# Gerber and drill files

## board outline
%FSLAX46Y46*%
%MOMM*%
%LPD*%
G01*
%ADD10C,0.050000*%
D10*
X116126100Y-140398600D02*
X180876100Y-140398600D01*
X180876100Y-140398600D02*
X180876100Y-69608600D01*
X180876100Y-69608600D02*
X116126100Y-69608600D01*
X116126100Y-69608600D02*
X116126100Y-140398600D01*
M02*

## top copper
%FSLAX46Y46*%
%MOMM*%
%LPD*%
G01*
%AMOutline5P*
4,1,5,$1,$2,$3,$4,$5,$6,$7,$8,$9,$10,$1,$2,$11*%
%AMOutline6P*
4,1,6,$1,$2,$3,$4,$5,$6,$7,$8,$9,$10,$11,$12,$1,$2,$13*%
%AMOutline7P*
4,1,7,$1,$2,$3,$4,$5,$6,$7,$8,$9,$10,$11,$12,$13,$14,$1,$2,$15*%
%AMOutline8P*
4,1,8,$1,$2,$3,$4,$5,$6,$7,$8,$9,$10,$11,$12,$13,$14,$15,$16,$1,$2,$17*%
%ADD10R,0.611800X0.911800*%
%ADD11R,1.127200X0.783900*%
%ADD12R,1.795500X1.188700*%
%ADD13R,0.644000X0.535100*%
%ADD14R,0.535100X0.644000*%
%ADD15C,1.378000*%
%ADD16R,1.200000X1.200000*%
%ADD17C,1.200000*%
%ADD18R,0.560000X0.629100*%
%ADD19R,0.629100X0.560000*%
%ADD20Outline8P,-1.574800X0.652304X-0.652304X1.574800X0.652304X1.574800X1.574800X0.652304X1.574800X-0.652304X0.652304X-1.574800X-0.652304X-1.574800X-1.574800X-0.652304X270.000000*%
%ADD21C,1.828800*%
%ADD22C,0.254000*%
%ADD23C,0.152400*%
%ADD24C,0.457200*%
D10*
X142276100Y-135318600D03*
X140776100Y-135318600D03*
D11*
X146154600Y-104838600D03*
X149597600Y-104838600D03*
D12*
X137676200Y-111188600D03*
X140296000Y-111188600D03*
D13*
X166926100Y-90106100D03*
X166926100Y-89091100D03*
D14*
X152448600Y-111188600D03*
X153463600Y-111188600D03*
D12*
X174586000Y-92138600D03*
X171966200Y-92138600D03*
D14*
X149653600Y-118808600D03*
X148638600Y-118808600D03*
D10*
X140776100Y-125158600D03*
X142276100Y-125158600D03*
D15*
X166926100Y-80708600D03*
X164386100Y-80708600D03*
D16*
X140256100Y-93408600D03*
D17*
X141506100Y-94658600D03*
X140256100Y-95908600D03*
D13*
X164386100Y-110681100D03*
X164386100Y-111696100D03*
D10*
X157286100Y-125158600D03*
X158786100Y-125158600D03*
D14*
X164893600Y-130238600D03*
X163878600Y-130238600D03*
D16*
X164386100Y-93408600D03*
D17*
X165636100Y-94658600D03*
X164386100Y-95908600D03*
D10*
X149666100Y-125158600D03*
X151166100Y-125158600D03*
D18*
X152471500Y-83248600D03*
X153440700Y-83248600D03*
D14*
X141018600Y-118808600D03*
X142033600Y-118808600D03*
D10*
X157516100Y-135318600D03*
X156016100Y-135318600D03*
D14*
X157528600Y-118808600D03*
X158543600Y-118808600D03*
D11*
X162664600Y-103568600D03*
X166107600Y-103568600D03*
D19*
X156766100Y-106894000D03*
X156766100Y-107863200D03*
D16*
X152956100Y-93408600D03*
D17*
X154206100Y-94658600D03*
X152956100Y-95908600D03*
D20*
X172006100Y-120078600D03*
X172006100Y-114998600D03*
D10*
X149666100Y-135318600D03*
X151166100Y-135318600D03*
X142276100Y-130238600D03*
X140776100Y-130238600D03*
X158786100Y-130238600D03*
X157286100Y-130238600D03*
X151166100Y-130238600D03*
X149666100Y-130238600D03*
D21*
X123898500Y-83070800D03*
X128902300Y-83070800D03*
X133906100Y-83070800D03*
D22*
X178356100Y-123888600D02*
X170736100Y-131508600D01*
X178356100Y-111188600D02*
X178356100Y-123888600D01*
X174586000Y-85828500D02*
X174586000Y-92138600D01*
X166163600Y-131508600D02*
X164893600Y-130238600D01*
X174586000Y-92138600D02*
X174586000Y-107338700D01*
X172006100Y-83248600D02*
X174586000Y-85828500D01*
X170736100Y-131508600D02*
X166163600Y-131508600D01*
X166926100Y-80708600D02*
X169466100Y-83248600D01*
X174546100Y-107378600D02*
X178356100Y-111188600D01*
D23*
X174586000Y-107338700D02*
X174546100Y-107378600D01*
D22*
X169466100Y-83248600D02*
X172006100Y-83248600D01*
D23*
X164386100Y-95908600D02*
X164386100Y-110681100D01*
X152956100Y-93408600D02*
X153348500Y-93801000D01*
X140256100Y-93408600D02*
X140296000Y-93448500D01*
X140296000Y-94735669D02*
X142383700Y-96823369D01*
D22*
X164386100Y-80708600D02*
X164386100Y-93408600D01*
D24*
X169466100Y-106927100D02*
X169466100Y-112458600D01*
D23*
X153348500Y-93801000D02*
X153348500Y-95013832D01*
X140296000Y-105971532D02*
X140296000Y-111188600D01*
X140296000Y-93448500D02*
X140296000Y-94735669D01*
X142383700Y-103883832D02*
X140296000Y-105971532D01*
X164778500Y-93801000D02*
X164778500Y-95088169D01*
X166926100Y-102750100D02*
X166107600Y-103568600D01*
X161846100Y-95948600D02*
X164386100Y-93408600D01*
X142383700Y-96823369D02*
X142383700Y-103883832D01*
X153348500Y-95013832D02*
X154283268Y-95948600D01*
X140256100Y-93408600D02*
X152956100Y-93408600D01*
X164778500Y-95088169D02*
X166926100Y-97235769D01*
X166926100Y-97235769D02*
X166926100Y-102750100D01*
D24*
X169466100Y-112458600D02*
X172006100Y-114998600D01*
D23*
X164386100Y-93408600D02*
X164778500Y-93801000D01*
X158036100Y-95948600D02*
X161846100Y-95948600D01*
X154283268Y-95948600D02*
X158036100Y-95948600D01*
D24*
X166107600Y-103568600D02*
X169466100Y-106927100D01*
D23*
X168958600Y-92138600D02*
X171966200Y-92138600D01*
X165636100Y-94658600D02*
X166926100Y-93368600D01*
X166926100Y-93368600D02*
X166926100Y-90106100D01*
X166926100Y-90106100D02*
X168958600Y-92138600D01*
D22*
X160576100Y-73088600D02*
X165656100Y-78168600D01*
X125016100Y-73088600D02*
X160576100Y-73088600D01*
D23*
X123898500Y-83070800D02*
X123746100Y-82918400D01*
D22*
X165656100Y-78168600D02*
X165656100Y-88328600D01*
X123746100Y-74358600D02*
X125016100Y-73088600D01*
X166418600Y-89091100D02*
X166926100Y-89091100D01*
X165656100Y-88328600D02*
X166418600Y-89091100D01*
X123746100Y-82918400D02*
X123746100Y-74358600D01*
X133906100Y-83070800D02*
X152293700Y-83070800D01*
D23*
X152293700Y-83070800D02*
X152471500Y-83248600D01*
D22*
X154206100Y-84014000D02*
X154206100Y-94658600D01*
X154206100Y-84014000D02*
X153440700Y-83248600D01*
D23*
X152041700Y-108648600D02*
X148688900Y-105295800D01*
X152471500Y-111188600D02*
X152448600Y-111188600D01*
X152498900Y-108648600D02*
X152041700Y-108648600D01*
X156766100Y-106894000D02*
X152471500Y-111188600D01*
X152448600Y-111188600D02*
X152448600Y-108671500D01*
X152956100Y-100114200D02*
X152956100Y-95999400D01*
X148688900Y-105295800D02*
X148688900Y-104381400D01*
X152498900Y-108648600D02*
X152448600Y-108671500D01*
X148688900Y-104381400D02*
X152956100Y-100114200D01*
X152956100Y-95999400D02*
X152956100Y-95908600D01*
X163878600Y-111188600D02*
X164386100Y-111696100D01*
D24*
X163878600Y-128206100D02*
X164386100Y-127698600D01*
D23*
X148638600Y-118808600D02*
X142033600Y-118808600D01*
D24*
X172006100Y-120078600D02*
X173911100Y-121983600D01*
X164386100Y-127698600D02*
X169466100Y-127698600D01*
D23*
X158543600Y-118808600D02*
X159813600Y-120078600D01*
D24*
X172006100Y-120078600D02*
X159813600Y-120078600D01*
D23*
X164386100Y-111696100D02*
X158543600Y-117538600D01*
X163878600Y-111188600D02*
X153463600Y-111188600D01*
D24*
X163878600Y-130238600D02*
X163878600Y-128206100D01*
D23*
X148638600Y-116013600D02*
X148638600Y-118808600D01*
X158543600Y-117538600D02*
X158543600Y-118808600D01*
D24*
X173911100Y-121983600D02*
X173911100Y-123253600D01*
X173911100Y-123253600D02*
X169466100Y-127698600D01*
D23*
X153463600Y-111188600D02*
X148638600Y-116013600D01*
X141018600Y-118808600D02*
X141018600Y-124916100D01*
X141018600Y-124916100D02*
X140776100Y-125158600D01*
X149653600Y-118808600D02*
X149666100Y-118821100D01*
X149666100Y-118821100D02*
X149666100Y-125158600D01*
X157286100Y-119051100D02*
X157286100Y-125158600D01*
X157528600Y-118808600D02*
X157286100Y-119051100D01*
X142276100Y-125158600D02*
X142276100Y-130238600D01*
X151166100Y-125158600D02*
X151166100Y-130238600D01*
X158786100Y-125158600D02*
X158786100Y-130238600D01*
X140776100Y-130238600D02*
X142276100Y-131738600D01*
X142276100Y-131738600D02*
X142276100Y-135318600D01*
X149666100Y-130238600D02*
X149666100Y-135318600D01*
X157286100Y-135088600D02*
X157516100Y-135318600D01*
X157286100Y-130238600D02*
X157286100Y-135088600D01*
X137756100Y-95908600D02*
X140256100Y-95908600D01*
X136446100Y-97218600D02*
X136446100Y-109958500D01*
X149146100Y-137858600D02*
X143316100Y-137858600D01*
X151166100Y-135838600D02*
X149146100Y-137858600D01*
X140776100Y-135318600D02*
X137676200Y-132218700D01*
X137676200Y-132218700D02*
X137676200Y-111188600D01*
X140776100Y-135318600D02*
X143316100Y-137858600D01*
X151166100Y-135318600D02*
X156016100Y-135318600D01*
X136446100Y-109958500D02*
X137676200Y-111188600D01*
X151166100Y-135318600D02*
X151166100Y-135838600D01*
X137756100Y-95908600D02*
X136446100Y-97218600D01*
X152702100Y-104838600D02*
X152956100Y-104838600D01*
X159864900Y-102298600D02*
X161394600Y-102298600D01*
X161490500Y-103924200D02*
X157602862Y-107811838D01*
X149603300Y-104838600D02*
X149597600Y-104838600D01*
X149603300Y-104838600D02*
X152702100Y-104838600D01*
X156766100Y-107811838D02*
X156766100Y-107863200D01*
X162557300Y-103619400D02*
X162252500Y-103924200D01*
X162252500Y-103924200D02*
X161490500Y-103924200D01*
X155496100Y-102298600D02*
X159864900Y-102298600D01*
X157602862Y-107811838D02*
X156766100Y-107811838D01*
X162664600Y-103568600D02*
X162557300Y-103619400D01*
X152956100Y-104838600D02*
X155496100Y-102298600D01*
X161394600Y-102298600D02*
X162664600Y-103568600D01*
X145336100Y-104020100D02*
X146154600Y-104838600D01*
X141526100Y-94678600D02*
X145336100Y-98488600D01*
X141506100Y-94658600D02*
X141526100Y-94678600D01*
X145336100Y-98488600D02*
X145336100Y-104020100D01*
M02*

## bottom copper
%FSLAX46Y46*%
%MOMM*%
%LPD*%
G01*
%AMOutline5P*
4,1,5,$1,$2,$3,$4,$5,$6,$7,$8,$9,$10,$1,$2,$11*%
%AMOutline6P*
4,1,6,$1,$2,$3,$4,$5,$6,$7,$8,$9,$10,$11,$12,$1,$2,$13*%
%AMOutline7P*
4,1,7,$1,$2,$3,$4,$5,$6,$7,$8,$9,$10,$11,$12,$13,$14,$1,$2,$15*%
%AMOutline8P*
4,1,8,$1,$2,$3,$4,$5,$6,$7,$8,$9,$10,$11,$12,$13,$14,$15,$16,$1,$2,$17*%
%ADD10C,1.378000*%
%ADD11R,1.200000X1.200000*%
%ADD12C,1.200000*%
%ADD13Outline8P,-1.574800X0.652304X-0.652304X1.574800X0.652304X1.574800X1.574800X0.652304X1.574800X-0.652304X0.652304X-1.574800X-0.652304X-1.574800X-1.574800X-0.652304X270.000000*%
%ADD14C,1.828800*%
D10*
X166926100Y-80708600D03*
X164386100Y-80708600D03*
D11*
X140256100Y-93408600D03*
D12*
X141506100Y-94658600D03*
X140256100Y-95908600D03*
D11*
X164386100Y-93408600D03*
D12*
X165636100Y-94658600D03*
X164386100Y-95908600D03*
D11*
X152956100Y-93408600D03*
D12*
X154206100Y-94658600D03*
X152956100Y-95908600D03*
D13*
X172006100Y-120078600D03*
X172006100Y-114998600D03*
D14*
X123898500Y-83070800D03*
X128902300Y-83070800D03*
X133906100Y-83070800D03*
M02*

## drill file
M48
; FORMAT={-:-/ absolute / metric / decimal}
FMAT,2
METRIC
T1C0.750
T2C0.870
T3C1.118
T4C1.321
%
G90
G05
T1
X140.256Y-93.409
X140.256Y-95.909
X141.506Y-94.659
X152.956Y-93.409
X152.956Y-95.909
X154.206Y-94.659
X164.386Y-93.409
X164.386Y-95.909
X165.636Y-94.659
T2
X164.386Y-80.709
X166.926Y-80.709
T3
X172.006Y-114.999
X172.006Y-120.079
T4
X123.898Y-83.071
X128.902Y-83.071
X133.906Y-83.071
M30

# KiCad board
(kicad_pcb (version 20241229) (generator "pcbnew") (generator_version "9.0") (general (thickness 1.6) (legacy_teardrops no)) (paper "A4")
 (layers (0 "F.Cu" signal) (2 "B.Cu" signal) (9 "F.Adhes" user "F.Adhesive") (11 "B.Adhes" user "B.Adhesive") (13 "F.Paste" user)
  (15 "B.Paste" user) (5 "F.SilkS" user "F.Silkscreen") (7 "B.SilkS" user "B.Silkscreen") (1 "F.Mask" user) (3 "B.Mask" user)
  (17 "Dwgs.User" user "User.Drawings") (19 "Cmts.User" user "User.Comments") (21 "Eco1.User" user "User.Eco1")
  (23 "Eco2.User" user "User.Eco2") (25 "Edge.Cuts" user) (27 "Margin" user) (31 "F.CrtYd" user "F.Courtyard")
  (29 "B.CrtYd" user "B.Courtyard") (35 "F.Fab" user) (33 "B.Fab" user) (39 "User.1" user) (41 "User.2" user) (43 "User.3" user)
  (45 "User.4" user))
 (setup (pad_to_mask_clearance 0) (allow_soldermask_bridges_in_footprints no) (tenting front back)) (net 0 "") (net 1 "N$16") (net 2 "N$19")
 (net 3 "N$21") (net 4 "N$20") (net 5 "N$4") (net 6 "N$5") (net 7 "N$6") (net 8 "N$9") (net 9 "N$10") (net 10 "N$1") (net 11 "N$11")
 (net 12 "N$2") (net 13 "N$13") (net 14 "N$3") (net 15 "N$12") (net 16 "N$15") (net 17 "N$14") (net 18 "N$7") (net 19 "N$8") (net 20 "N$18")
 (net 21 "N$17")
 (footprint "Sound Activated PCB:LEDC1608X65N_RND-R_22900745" (layer "F.Cu") (at 141.5261 135.3186)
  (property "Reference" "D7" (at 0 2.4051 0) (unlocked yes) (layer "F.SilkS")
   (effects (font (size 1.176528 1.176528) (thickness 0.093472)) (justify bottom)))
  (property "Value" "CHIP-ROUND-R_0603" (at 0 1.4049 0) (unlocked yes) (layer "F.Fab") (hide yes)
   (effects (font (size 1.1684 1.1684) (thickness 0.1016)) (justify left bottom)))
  (pad "A" smd rect (at 0.75 0) (size 0.6118 0.9118) (layers "F.Cu" "F.Mask" "F.Paste") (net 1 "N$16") (solder_mask_margin 0.1016)
   (solder_paste_margin 0) (thermal_bridge_angle 0))
  (pad "C" smd rect (at -0.75 0) (size 0.6118 0.9118) (layers "F.Cu" "F.Mask" "F.Paste") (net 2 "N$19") (solder_mask_margin 0.1016)
   (solder_paste_margin 0) (thermal_bridge_angle 0)))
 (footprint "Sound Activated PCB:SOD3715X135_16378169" (layer "F.Cu") (at 147.8761 104.8386)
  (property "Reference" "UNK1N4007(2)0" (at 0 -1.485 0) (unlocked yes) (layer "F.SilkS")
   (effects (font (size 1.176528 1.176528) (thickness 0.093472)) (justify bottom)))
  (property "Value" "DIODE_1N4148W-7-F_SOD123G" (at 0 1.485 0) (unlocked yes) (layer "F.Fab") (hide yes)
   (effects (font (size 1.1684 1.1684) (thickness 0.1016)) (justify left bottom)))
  (pad "1" smd rect (at -1.7215 0) (size 1.1272 0.7839) (layers "F.Cu" "F.Mask" "F.Paste") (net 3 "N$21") (solder_mask_margin 0.1016)
   (solder_paste_margin 0) (thermal_bridge_angle 0))
  (pad "2" smd rect (at 1.7215 0) (size 1.1272 0.7839) (layers "F.Cu" "F.Mask" "F.Paste") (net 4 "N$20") (solder_mask_margin 0.1016)
   (solder_paste_margin 0) (thermal_bridge_angle 0)))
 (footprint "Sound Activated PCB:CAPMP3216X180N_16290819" (layer "F.Cu") (at 138.9861 111.1886)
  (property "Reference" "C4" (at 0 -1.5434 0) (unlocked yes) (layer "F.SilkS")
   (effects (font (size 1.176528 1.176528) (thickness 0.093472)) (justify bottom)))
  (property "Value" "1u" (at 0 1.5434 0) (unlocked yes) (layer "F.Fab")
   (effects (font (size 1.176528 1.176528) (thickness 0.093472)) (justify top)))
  (pad "1" smd rect (at -1.3099 0) (size 1.7955 1.1887) (layers "F.Cu" "F.Mask" "F.Paste") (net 2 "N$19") (solder_mask_margin 0.1016)
   (solder_paste_margin 0) (thermal_bridge_angle 0))
  (pad "2" smd rect (at 1.3099 0) (size 1.7955 1.1887) (layers "F.Cu" "F.Mask" "F.Paste") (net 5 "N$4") (solder_mask_margin 0.1016)
   (solder_paste_margin 0) (thermal_bridge_angle 0)))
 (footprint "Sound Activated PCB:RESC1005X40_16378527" (layer "F.Cu") (at 166.9261 89.5986 90)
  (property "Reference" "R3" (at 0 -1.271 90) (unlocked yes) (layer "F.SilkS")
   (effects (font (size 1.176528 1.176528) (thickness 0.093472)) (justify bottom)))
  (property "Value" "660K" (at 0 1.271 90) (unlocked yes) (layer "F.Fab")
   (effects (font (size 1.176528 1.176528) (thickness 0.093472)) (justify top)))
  (pad "1" smd rect (at -0.5075 0 90) (size 0.5351 0.644) (layers "F.Cu" "F.Mask" "F.Paste") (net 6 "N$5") (solder_mask_margin 0.1016)
   (solder_paste_margin 0) (thermal_bridge_angle 0))
  (pad "2" smd rect (at 0.5075 0 90) (size 0.5351 0.644) (layers "F.Cu" "F.Mask" "F.Paste") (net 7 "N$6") (solder_mask_margin 0.1016)
   (solder_paste_margin 0) (thermal_bridge_angle 0)))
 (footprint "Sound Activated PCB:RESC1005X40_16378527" (layer "F.Cu") (at 152.9561 111.1886)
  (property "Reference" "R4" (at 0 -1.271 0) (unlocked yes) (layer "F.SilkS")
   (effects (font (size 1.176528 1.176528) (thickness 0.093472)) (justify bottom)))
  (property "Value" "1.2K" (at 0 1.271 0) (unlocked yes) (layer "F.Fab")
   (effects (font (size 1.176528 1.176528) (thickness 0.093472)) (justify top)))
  (pad "1" smd rect (at -0.5075 0) (size 0.5351 0.644) (layers "F.Cu" "F.Mask" "F.Paste") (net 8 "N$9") (solder_mask_margin 0.1016)
   (solder_paste_margin 0) (thermal_bridge_angle 0))
  (pad "2" smd rect (at 0.5075 0) (size 0.5351 0.644) (layers "F.Cu" "F.Mask" "F.Paste") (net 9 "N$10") (solder_mask_margin 0.1016)
   (solder_paste_margin 0) (thermal_bridge_angle 0)))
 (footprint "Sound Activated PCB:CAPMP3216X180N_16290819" (layer "F.Cu") (at 173.2761 92.1386 180)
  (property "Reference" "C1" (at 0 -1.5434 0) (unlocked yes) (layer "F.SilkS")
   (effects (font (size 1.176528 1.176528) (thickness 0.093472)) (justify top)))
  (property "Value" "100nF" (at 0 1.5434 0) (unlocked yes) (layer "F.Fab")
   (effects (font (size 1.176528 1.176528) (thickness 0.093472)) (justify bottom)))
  (pad "1" smd rect (at -1.3099 0 180) (size 1.7955 1.1887) (layers "F.Cu" "F.Mask" "F.Paste") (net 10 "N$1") (solder_mask_margin 0.1016)
   (solder_paste_margin 0) (thermal_bridge_angle 0))
  (pad "2" smd rect (at 1.3099 0 180) (size 1.7955 1.1887) (layers "F.Cu" "F.Mask" "F.Paste") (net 6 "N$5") (solder_mask_margin 0.1016)
   (solder_paste_margin 0) (thermal_bridge_angle 0)))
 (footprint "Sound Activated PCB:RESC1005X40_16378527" (layer "F.Cu") (at 149.1461 118.8086 180)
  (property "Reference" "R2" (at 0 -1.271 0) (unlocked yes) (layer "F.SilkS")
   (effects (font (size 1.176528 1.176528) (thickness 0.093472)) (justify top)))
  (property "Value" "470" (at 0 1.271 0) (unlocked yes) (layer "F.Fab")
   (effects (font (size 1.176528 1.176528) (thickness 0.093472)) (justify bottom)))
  (pad "1" smd rect (at -0.5075 0 180) (size 0.5351 0.644) (layers "F.Cu" "F.Mask" "F.Paste") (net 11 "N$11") (solder_mask_margin 0.1016)
   (solder_paste_margin 0) (thermal_bridge_angle 0))
  (pad "2" smd rect (at 0.5075 0 180) (size 0.5351 0.644) (layers "F.Cu" "F.Mask" "F.Paste") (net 9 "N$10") (solder_mask_margin 0.1016)
   (solder_paste_margin 0) (thermal_bridge_angle 0)))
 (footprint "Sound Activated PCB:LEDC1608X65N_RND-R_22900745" (layer "F.Cu") (at 141.5261 125.1586 180)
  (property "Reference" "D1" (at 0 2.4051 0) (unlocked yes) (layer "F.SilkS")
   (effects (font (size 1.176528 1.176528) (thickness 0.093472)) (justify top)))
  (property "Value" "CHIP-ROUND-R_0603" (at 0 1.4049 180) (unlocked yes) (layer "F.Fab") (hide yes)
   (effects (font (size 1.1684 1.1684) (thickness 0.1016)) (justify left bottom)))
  (pad "A" smd rect (at 0.75 0 180) (size 0.6118 0.9118) (layers "F.Cu" "F.Mask" "F.Paste") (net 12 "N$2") (solder_mask_margin 0.1016)
   (solder_paste_margin 0) (thermal_bridge_angle 0))
  (pad "C" smd rect (at -0.75 0 180) (size 0.6118 0.9118) (layers "F.Cu" "F.Mask" "F.Paste") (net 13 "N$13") (solder_mask_margin 0.1016)
   (solder_paste_margin 0) (thermal_bridge_angle 0)))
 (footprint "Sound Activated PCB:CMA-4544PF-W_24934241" (layer "F.Cu") (at 164.3861 80.7086 90)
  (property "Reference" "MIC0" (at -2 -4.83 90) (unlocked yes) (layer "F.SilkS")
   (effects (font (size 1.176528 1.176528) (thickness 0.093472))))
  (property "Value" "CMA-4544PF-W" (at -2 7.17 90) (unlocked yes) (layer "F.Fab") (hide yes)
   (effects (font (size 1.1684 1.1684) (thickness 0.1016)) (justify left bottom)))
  (pad "1" thru_hole circle (at 0 2.54 90) (size 1.378 1.378) (drill 0.87) (layers "*.Cu" "*.Mask") (remove_unused_layers no) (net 10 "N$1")
   (solder_mask_margin 0.1016) (thermal_bridge_angle 0))
  (pad "2" thru_hole circle (at 0 0 90) (size 1.378 1.378) (drill 0.87) (layers "*.Cu" "*.Mask") (remove_unused_layers no) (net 5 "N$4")
   (solder_mask_margin 0.1016) (thermal_bridge_angle 0)))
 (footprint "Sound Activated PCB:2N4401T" (layer "F.Cu") (at 140.2561 93.4086 -90)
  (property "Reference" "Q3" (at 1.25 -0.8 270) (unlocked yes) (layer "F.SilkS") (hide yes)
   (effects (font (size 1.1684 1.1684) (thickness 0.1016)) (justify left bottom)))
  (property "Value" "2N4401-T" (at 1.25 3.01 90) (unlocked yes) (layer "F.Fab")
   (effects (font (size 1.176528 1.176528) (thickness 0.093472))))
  (pad "1" thru_hole rect (at 0 0 270) (size 1.2 1.2) (drill 0.75) (layers "*.Cu" "*.Mask") (remove_unused_layers no) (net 5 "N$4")
   (solder_mask_margin 0.1016) (thermal_bridge_angle 0))
  (pad "2" thru_hole circle (at 1.25 -1.25 270) (size 1.2 1.2) (drill 0.75) (layers "*.Cu" "*.Mask") (remove_unused_layers no)
   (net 3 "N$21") (solder_mask_margin 0.1016) (thermal_bridge_angle 0))
  (pad "3" thru_hole circle (at 2.5 0 270) (size 1.2 1.2) (drill 0.75) (layers "*.Cu" "*.Mask") (remove_unused_layers no) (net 2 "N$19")
   (solder_mask_margin 0.1016) (thermal_bridge_angle 0)))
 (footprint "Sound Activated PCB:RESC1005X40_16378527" (layer "F.Cu") (at 164.3861 111.1886 -90)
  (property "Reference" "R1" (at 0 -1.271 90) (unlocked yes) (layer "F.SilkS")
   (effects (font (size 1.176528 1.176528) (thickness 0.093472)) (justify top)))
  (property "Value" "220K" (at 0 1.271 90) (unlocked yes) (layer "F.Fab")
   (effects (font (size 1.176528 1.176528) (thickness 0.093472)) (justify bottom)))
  (pad "1" smd rect (at -0.5075 0 270) (size 0.5351 0.644) (layers "F.Cu" "F.Mask" "F.Paste") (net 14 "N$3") (solder_mask_margin 0.1016)
   (solder_paste_margin 0) (thermal_bridge_angle 0))
  (pad "2" smd rect (at 0.5075 0 270) (size 0.5351 0.644) (layers "F.Cu" "F.Mask" "F.Paste") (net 9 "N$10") (solder_mask_margin 0.1016)
   (solder_paste_margin 0) (thermal_bridge_angle 0)))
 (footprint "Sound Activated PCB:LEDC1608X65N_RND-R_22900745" (layer "F.Cu") (at 158.0361 125.1586 180)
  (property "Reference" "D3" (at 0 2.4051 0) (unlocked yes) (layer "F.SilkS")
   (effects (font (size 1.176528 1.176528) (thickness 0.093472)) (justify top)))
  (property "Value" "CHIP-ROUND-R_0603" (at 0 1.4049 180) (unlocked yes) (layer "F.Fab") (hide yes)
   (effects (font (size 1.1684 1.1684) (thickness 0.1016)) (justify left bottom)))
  (pad "A" smd rect (at 0.75 0 180) (size 0.6118 0.9118) (layers "F.Cu" "F.Mask" "F.Paste") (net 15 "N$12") (solder_mask_margin 0.1016)
   (solder_paste_margin 0) (thermal_bridge_angle 0))
  (pad "C" smd rect (at -0.75 0 180) (size 0.6118 0.9118) (layers "F.Cu" "F.Mask" "F.Paste") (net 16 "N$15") (solder_mask_margin 0.1016)
   (solder_paste_margin 0) (thermal_bridge_angle 0)))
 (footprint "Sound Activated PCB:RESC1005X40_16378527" (layer "F.Cu") (at 164.3861 130.2386 180)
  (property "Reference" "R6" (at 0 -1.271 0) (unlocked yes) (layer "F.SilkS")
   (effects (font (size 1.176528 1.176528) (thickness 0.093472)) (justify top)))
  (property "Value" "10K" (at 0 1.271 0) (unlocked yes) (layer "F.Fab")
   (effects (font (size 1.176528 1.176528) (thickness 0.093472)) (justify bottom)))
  (pad "1" smd rect (at -0.5075 0 180) (size 0.5351 0.644) (layers "F.Cu" "F.Mask" "F.Paste") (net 10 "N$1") (solder_mask_margin 0.1016)
   (solder_paste_margin 0) (thermal_bridge_angle 0))
  (pad "2" smd rect (at 0.5075 0 180) (size 0.5351 0.644) (layers "F.Cu" "F.Mask" "F.Paste") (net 9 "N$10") (solder_mask_margin 0.1016)
   (solder_paste_margin 0) (thermal_bridge_angle 0)))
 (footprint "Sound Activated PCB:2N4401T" (layer "F.Cu") (at 164.3861 93.4086 -90)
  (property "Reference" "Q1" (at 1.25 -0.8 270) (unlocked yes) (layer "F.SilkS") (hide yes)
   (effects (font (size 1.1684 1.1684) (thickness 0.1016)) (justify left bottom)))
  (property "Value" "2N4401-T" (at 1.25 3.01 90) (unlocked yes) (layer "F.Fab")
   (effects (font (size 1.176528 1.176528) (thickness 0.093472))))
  (pad "1" thru_hole rect (at 0 0 270) (size 1.2 1.2) (drill 0.75) (layers "*.Cu" "*.Mask") (remove_unused_layers no) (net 5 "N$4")
   (solder_mask_margin 0.1016) (thermal_bridge_angle 0))
  (pad "2" thru_hole circle (at 1.25 -1.25 270) (size 1.2 1.2) (drill 0.75) (layers "*.Cu" "*.Mask") (remove_unused_layers no) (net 6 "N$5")
   (solder_mask_margin 0.1016) (thermal_bridge_angle 0))
  (pad "3" thru_hole circle (at 2.5 0 270) (size 1.2 1.2) (drill 0.75) (layers "*.Cu" "*.Mask") (remove_unused_layers no) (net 14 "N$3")
   (solder_mask_margin 0.1016) (thermal_bridge_angle 0)))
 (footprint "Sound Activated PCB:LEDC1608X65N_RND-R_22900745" (layer "F.Cu") (at 150.4161 125.1586 180)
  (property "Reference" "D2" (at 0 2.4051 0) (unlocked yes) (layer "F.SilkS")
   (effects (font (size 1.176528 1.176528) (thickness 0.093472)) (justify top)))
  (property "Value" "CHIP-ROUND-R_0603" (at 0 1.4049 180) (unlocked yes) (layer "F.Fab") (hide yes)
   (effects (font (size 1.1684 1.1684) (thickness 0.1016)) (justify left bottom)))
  (pad "A" smd rect (at 0.75 0 180) (size 0.6118 0.9118) (layers "F.Cu" "F.Mask" "F.Paste") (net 11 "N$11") (solder_mask_margin 0.1016)
   (solder_paste_margin 0) (thermal_bridge_angle 0))
  (pad "C" smd rect (at -0.75 0 180) (size 0.6118 0.9118) (layers "F.Cu" "F.Mask" "F.Paste") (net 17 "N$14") (solder_mask_margin 0.1016)
   (solder_paste_margin 0) (thermal_bridge_angle 0)))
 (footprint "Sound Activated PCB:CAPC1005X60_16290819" (layer "F.Cu") (at 152.9561 83.2486)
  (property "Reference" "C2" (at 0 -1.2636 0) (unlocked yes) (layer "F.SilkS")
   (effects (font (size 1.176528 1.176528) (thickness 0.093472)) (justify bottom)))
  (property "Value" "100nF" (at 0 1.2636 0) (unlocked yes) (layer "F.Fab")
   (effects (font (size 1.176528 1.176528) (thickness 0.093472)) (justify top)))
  (pad "1" smd rect (at -0.4846 0) (size 0.56 0.6291) (layers "F.Cu" "F.Mask" "F.Paste") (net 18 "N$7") (solder_mask_margin 0.1016)
   (solder_paste_margin 0) (thermal_bridge_angle 0))
  (pad "2" smd rect (at 0.4846 0) (size 0.56 0.6291) (layers "F.Cu" "F.Mask" "F.Paste") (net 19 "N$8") (solder_mask_margin 0.1016)
   (solder_paste_margin 0) (thermal_bridge_angle 0)))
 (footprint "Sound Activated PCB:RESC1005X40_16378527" (layer "F.Cu") (at 141.5261 118.8086)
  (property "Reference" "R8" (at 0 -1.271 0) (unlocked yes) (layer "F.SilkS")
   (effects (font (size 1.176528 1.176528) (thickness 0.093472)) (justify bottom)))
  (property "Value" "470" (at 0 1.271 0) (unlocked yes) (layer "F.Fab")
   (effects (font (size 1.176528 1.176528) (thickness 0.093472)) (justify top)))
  (pad "1" smd rect (at -0.5075 0) (size 0.5351 0.644) (layers "F.Cu" "F.Mask" "F.Paste") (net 12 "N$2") (solder_mask_margin 0.1016)
   (solder_paste_margin 0) (thermal_bridge_angle 0))
  (pad "2" smd rect (at 0.5075 0) (size 0.5351 0.644) (layers "F.Cu" "F.Mask" "F.Paste") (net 9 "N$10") (solder_mask_margin 0.1016)
   (solder_paste_margin 0) (thermal_bridge_angle 0)))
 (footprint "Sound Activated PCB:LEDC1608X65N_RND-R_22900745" (layer "F.Cu") (at 156.7661 135.3186)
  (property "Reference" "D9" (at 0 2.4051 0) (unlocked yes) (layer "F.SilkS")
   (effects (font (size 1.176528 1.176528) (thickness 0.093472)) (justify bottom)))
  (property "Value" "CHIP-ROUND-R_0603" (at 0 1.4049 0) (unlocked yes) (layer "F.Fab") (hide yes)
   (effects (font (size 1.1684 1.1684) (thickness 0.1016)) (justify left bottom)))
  (pad "A" smd rect (at 0.75 0) (size 0.6118 0.9118) (layers "F.Cu" "F.Mask" "F.Paste") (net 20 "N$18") (solder_mask_margin 0.1016)
   (solder_paste_margin 0) (thermal_bridge_angle 0))
  (pad "C" smd rect (at -0.75 0) (size 0.6118 0.9118) (layers "F.Cu" "F.Mask" "F.Paste") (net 2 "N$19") (solder_mask_margin 0.1016)
   (solder_paste_margin 0) (thermal_bridge_angle 0)))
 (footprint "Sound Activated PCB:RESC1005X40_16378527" (layer "F.Cu") (at 158.0361 118.8086)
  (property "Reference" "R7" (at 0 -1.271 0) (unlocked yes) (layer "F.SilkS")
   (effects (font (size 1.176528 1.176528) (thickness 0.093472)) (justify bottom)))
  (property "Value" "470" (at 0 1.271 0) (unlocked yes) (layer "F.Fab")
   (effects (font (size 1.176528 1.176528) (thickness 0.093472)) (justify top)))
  (pad "1" smd rect (at -0.5075 0) (size 0.5351 0.644) (layers "F.Cu" "F.Mask" "F.Paste") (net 15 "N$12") (solder_mask_margin 0.1016)
   (solder_paste_margin 0) (thermal_bridge_angle 0))
  (pad "2" smd rect (at 0.5075 0) (size 0.5351 0.644) (layers "F.Cu" "F.Mask" "F.Paste") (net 9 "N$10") (solder_mask_margin 0.1016)
   (solder_paste_margin 0) (thermal_bridge_angle 0)))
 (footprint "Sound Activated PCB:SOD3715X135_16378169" (layer "F.Cu") (at 164.3861 103.5686)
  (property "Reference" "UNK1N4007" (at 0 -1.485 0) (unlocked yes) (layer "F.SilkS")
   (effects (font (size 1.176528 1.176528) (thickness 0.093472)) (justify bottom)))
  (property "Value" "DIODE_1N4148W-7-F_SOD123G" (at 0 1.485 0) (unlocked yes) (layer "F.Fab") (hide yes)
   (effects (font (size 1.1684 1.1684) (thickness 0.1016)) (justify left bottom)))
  (pad "1" smd rect (at -1.7215 0) (size 1.1272 0.7839) (layers "F.Cu" "F.Mask" "F.Paste") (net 4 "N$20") (solder_mask_margin 0.1016)
   (solder_paste_margin 0) (thermal_bridge_angle 0))
  (pad "2" smd rect (at 1.7215 0) (size 1.1272 0.7839) (layers "F.Cu" "F.Mask" "F.Paste") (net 5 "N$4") (solder_mask_margin 0.1016)
   (solder_paste_margin 0) (thermal_bridge_angle 0)))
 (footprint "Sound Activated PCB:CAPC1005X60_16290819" (layer "F.Cu") (at 156.7661 107.3786 -90)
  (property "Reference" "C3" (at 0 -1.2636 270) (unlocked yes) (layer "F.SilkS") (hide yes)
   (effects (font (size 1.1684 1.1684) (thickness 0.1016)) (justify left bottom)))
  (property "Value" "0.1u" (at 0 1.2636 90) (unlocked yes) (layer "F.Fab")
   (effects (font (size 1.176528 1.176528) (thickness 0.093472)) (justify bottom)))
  (pad "1" smd rect (at -0.4846 0 270) (size 0.56 0.6291) (layers "F.Cu" "F.Mask" "F.Paste") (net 8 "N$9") (solder_mask_margin 0.1016)
   (solder_paste_margin 0) (thermal_bridge_angle 0))
  (pad "2" smd rect (at 0.4846 0 270) (size 0.56 0.6291) (layers "F.Cu" "F.Mask" "F.Paste") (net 4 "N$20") (solder_mask_margin 0.1016)
   (solder_paste_margin 0) (thermal_bridge_angle 0)))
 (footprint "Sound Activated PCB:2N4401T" (layer "F.Cu") (at 152.9561 93.4086 -90)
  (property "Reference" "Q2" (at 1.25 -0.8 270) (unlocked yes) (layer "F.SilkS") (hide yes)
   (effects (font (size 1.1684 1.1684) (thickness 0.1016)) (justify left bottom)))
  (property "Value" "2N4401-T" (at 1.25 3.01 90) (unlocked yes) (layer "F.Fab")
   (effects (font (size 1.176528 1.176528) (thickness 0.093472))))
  (pad "1" thru_hole rect (at 0 0 270) (size 1.2 1.2) (drill 0.75) (layers "*.Cu" "*.Mask") (remove_unused_layers no) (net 5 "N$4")
   (solder_mask_margin 0.1016) (thermal_bridge_angle 0))
  (pad "2" thru_hole circle (at 1.25 -1.25 270) (size 1.2 1.2) (drill 0.75) (layers "*.Cu" "*.Mask") (remove_unused_layers no)
   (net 19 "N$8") (solder_mask_margin 0.1016) (thermal_bridge_angle 0))
  (pad "3" thru_hole circle (at 2.5 0 270) (size 1.2 1.2) (drill 0.75) (layers "*.Cu" "*.Mask") (remove_unused_layers no) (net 8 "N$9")
   (solder_mask_margin 0.1016) (thermal_bridge_angle 0)))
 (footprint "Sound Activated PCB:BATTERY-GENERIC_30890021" (layer "F.Cu") (at 172.0061 117.5386 -90)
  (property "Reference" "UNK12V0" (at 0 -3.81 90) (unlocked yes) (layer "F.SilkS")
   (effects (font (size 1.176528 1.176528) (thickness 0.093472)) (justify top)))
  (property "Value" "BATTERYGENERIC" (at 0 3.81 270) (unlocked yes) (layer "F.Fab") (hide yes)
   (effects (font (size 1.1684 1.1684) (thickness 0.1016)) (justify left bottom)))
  (pad "+" thru_hole roundrect (at 2.54 0 270) (size 3.1496 3.1496) (drill 1.1176) (layers "*.Cu" "*.Mask") (remove_unused_layers no)
   (roundrect_rratio 0.25) (chamfer_ratio 0.2928932188) (chamfer top_left top_right bottom_left bottom_right) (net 9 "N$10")
   (solder_mask_margin 0.1016) (thermal_bridge_angle 0))
  (pad "-" thru_hole roundrect (at -2.54 0 270) (size 3.1496 3.1496) (drill 1.1176) (layers "*.Cu" "*.Mask") (remove_unused_layers no)
   (roundrect_rratio 0.25) (chamfer_ratio 0.2928932188) (chamfer top_left top_right bottom_left bottom_right) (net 5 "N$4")
   (solder_mask_margin 0.1016) (thermal_bridge_angle 0)))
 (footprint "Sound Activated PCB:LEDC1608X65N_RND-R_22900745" (layer "F.Cu") (at 150.4161 135.3186 180)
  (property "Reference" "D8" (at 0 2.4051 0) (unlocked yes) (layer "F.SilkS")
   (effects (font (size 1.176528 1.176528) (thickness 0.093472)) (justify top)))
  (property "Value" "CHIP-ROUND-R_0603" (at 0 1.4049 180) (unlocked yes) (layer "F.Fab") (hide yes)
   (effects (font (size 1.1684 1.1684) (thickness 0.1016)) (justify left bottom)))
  (pad "A" smd rect (at 0.75 0 180) (size 0.6118 0.9118) (layers "F.Cu" "F.Mask" "F.Paste") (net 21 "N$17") (solder_mask_margin 0.1016)
   (solder_paste_margin 0) (thermal_bridge_angle 0))
  (pad "C" smd rect (at -0.75 0 180) (size 0.6118 0.9118) (layers "F.Cu" "F.Mask" "F.Paste") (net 2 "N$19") (solder_mask_margin 0.1016)
   (solder_paste_margin 0) (thermal_bridge_angle 0)))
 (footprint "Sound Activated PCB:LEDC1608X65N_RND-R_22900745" (layer "F.Cu") (at 141.5261 130.2386)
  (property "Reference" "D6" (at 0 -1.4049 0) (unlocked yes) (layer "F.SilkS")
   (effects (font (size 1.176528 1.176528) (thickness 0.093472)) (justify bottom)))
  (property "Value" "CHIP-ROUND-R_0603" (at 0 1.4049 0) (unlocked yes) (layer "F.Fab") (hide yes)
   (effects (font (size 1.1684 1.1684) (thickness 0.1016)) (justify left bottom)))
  (pad "A" smd rect (at 0.75 0) (size 0.6118 0.9118) (layers "F.Cu" "F.Mask" "F.Paste") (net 13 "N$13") (solder_mask_margin 0.1016)
   (solder_paste_margin 0) (thermal_bridge_angle 0))
  (pad "C" smd rect (at -0.75 0) (size 0.6118 0.9118) (layers "F.Cu" "F.Mask" "F.Paste") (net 1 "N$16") (solder_mask_margin 0.1016)
   (solder_paste_margin 0) (thermal_bridge_angle 0)))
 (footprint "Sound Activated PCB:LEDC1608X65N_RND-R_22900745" (layer "F.Cu") (at 158.0361 130.2386)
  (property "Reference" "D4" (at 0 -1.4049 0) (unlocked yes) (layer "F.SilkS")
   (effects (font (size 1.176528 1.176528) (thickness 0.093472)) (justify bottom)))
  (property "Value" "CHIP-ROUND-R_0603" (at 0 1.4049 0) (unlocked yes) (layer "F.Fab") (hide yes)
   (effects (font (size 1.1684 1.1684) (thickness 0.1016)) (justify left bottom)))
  (pad "A" smd rect (at 0.75 0) (size 0.6118 0.9118) (layers "F.Cu" "F.Mask" "F.Paste") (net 16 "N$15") (solder_mask_margin 0.1016)
   (solder_paste_margin 0) (thermal_bridge_angle 0))
  (pad "C" smd rect (at -0.75 0) (size 0.6118 0.9118) (layers "F.Cu" "F.Mask" "F.Paste") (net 20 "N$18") (solder_mask_margin 0.1016)
   (solder_paste_margin 0) (thermal_bridge_angle 0)))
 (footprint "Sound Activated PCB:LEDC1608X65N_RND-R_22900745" (layer "F.Cu") (at 150.4161 130.2386)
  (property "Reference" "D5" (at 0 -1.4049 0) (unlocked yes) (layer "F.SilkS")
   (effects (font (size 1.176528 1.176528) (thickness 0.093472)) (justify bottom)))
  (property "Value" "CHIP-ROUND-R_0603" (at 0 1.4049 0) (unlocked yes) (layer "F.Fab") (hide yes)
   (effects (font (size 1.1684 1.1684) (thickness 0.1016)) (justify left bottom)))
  (pad "A" smd rect (at 0.75 0) (size 0.6118 0.9118) (layers "F.Cu" "F.Mask" "F.Paste") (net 17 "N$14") (solder_mask_margin 0.1016)
   (solder_paste_margin 0) (thermal_bridge_angle 0))
  (pad "C" smd rect (at -0.75 0) (size 0.6118 0.9118) (layers "F.Cu" "F.Mask" "F.Paste") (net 21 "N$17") (solder_mask_margin 0.1016)
   (solder_paste_margin 0) (thermal_bridge_angle 0)))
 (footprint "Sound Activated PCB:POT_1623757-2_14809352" (layer "F.Cu") (at 133.9061 70.5486)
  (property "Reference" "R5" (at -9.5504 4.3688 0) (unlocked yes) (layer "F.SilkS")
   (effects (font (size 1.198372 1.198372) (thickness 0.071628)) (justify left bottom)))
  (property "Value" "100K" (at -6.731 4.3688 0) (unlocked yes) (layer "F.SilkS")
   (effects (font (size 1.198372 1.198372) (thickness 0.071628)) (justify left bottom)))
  (pad "1" thru_hole circle (at -10.0076 12.5222) (size 1.8288 1.8288) (drill 1.3208) (layers "*.Cu" "*.Mask") (remove_unused_layers no)
   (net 7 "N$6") (solder_mask_margin 0.1016) (thermal_bridge_angle 0))
  (pad "2" thru_hole circle (at -5.0038 12.5222) (size 1.8288 1.8288) (drill 1.3208) (layers "*.Cu" "*.Mask") (remove_unused_layers no)
   (solder_mask_margin 0.1016) (thermal_bridge_angle 0))
  (pad "3" thru_hole circle (at 0 12.5222) (size 1.8288 1.8288) (drill 1.3208) (layers "*.Cu" "*.Mask") (remove_unused_layers no)
   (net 18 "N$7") (solder_mask_margin 0.1016) (thermal_bridge_angle 0)))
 (gr_line (start 116.1261 140.3986) (end 180.8761 140.3986) (stroke (width 0.05) (type solid)) (layer "Edge.Cuts"))
 (gr_line (start 180.8761 140.3986) (end 180.8761 69.6086) (stroke (width 0.05) (type solid)) (layer "Edge.Cuts"))
 (gr_line (start 180.8761 69.6086) (end 116.1261 69.6086) (stroke (width 0.05) (type solid)) (layer "Edge.Cuts"))
 (gr_line (start 116.1261 69.6086) (end 116.1261 140.3986) (stroke (width 0.05) (type solid)) (layer "Edge.Cuts"))
 (segment (start 178.3561 123.8886) (end 170.7361 131.5086) (width 0.254) (layer "F.Cu") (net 10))
 (segment (start 178.3561 111.1886) (end 178.3561 123.8886) (width 0.254) (layer "F.Cu") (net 10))
 (segment (start 174.586 85.8285) (end 174.586 92.1386) (width 0.254) (layer "F.Cu") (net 10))
 (segment (start 166.1636 131.5086) (end 164.8936 130.2386) (width 0.254) (layer "F.Cu") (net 10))
 (segment (start 174.586 92.1386) (end 174.586 107.3387) (width 0.254) (layer "F.Cu") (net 10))
 (segment (start 172.0061 83.2486) (end 174.586 85.8285) (width 0.254) (layer "F.Cu") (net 10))
 (segment (start 170.7361 131.5086) (end 166.1636 131.5086) (width 0.254) (layer "F.Cu") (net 10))
 (segment (start 166.9261 80.7086) (end 169.4661 83.2486) (width 0.254) (layer "F.Cu") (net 10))
 (segment (start 174.5461 107.3786) (end 178.3561 111.1886) (width 0.254) (layer "F.Cu") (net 10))
 (segment (start 174.586 107.3387) (end 174.5461 107.3786) (width 0.1524) (layer "F.Cu") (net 10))
 (segment (start 169.4661 83.2486) (end 172.0061 83.2486) (width 0.254) (layer "F.Cu") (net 10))
 (segment (start 164.3861 95.9086) (end 164.3861 110.6811) (width 0.1524) (layer "F.Cu") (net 14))
 (segment (start 152.9561 93.4086) (end 153.3485 93.801) (width 0.1524) (layer "F.Cu") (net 5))
 (segment (start 140.2561 93.4086) (end 140.296 93.4485) (width 0.1524) (layer "F.Cu") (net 5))
 (segment (start 140.296 94.735669) (end 142.3837 96.823369) (width 0.1524) (layer "F.Cu") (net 5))
 (segment (start 164.3861 80.7086) (end 164.3861 93.4086) (width 0.254) (layer "F.Cu") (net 5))
 (segment (start 169.4661 106.9271) (end 169.4661 112.4586) (width 0.4572) (layer "F.Cu") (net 5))
 (segment (start 153.3485 93.801) (end 153.3485 95.013832) (width 0.1524) (layer "F.Cu") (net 5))
 (segment (start 140.296 105.971532) (end 140.296 111.1886) (width 0.1524) (layer "F.Cu") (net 5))
 (segment (start 140.296 93.4485) (end 140.296 94.735669) (width 0.1524) (layer "F.Cu") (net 5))
 (segment (start 142.3837 103.883832) (end 140.296 105.971532) (width 0.1524) (layer "F.Cu") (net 5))
 (segment (start 164.7785 93.801) (end 164.7785 95.088169) (width 0.1524) (layer "F.Cu") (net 5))
 (segment (start 166.9261 102.7501) (end 166.1076 103.5686) (width 0.1524) (layer "F.Cu") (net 5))
 (segment (start 161.8461 95.9486) (end 164.3861 93.4086) (width 0.1524) (layer "F.Cu") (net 5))
 (segment (start 142.3837 96.823369) (end 142.3837 103.883832) (width 0.1524) (layer "F.Cu") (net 5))
 (segment (start 153.3485 95.013832) (end 154.283268 95.9486) (width 0.1524) (layer "F.Cu") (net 5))
 (segment (start 140.2561 93.4086) (end 152.9561 93.4086) (width 0.1524) (layer "F.Cu") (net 5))
 (segment (start 164.7785 95.088169) (end 166.9261 97.235769) (width 0.1524) (layer "F.Cu") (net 5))
 (segment (start 166.9261 97.235769) (end 166.9261 102.7501) (width 0.1524) (layer "F.Cu") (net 5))
 (segment (start 169.4661 112.4586) (end 172.0061 114.9986) (width 0.4572) (layer "F.Cu") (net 5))
 (segment (start 164.3861 93.4086) (end 164.7785 93.801) (width 0.1524) (layer "F.Cu") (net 5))
 (segment (start 158.0361 95.9486) (end 161.8461 95.9486) (width 0.1524) (layer "F.Cu") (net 5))
 (segment (start 154.283268 95.9486) (end 158.0361 95.9486) (width 0.1524) (layer "F.Cu") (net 5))
 (segment (start 166.1076 103.5686) (end 169.4661 106.9271) (width 0.4572) (layer "F.Cu") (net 5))
 (segment (start 168.9586 92.1386) (end 171.9662 92.1386) (width 0.1524) (layer "F.Cu") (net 6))
 (segment (start 165.6361 94.6586) (end 166.9261 93.3686) (width 0.1524) (layer "F.Cu") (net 6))
 (segment (start 166.9261 93.3686) (end 166.9261 90.1061) (width 0.1524) (layer "F.Cu") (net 6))
 (segment (start 166.9261 90.1061) (end 168.9586 92.1386) (width 0.1524) (layer "F.Cu") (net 6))
 (segment (start 160.5761 73.0886) (end 165.6561 78.1686) (width 0.254) (layer "F.Cu") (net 7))
 (segment (start 125.0161 73.0886) (end 160.5761 73.0886) (width 0.254) (layer "F.Cu") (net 7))
 (segment (start 123.8985 83.0708) (end 123.7461 82.9184) (width 0.1524) (layer "F.Cu") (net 7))
 (segment (start 165.6561 78.1686) (end 165.6561 88.3286) (width 0.254) (layer "F.Cu") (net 7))
 (segment (start 123.7461 74.3586) (end 125.0161 73.0886) (width 0.254) (layer "F.Cu") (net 7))
 (segment (start 166.4186 89.0911) (end 166.9261 89.0911) (width 0.254) (layer "F.Cu") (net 7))
 (segment (start 165.6561 88.3286) (end 166.4186 89.0911) (width 0.254) (layer "F.Cu") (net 7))
 (segment (start 123.7461 82.9184) (end 123.7461 74.3586) (width 0.254) (layer "F.Cu") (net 7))
 (segment (start 133.9061 83.0708) (end 152.2937 83.0708) (width 0.254) (layer "F.Cu") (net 18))
 (segment (start 152.2937 83.0708) (end 152.4715 83.2486) (width 0.1524) (layer "F.Cu") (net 18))
 (segment (start 154.2061 84.014) (end 154.2061 94.6586) (width 0.254) (layer "F.Cu") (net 19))
 (segment (start 154.2061 84.014) (end 153.4407 83.2486) (width 0.254) (layer "F.Cu") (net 19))
 (segment (start 152.0417 108.6486) (end 148.6889 105.2958) (width 0.1524) (layer "F.Cu") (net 8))
 (segment (start 152.4715 111.1886) (end 152.4486 111.1886) (width 0.1524) (layer "F.Cu") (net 8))
 (segment (start 152.4989 108.6486) (end 152.0417 108.6486) (width 0.1524) (layer "F.Cu") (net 8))
 (segment (start 156.7661 106.894) (end 152.4715 111.1886) (width 0.1524) (layer "F.Cu") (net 8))
 (segment (start 152.4486 111.1886) (end 152.4486 108.6715) (width 0.1524) (layer "F.Cu") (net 8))
 (segment (start 152.9561 100.1142) (end 152.9561 95.9994) (width 0.1524) (layer "F.Cu") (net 8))
 (segment (start 148.6889 105.2958) (end 148.6889 104.3814) (width 0.1524) (layer "F.Cu") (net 8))
 (segment (start 152.4989 108.6486) (end 152.4486 108.6715) (width 0.1524) (layer "F.Cu") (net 8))
 (segment (start 148.6889 104.3814) (end 152.9561 100.1142) (width 0.1524) (layer "F.Cu") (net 8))
 (segment (start 152.9561 95.9994) (end 152.9561 95.9086) (width 0.1524) (layer "F.Cu") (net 8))
 (segment (start 163.8786 111.1886) (end 164.3861 111.6961) (width 0.1524) (layer "F.Cu") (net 9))
 (segment (start 163.8786 128.2061) (end 164.3861 127.6986) (width 0.4572) (layer "F.Cu") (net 9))
 (segment (start 148.6386 118.8086) (end 142.0336 118.8086) (width 0.1524) (layer "F.Cu") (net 9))
 (segment (start 172.0061 120.0786) (end 173.9111 121.9836) (width 0.4572) (layer "F.Cu") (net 9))
 (segment (start 164.3861 127.6986) (end 169.4661 127.6986) (width 0.4572) (layer "F.Cu") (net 9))
 (segment (start 158.5436 118.8086) (end 159.8136 120.0786) (width 0.1524) (layer "F.Cu") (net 9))
 (segment (start 172.0061 120.0786) (end 159.8136 120.0786) (width 0.4572) (layer "F.Cu") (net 9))
 (segment (start 164.3861 111.6961) (end 158.5436 117.5386) (width 0.1524) (layer "F.Cu") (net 9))
 (segment (start 163.8786 111.1886) (end 153.4636 111.1886) (width 0.1524) (layer "F.Cu") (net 9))
 (segment (start 163.8786 130.2386) (end 163.8786 128.2061) (width 0.4572) (layer "F.Cu") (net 9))
 (segment (start 148.6386 116.0136) (end 148.6386 118.8086) (width 0.1524) (layer "F.Cu") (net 9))
 (segment (start 158.5436 117.5386) (end 158.5436 118.8086) (width 0.1524) (layer "F.Cu") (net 9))
 (segment (start 173.9111 121.9836) (end 173.9111 123.2536) (width 0.4572) (layer "F.Cu") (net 9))
 (segment (start 173.9111 123.2536) (end 169.4661 127.6986) (width 0.4572) (layer "F.Cu") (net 9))
 (segment (start 153.4636 111.1886) (end 148.6386 116.0136) (width 0.1524) (layer "F.Cu") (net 9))
 (segment (start 141.0186 118.8086) (end 141.0186 124.9161) (width 0.1524) (layer "F.Cu") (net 12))
 (segment (start 141.0186 124.9161) (end 140.7761 125.1586) (width 0.1524) (layer "F.Cu") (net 12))
 (segment (start 149.6536 118.8086) (end 149.6661 118.8211) (width 0.1524) (layer "F.Cu") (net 11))
 (segment (start 149.6661 118.8211) (end 149.6661 125.1586) (width 0.1524) (layer "F.Cu") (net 11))
 (segment (start 157.2861 119.0511) (end 157.2861 125.1586) (width 0.1524) (layer "F.Cu") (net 15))
 (segment (start 157.5286 118.8086) (end 157.2861 119.0511) (width 0.1524) (layer "F.Cu") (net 15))
 (segment (start 142.2761 125.1586) (end 142.2761 130.2386) (width 0.1524) (layer "F.Cu") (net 13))
 (segment (start 151.1661 125.1586) (end 151.1661 130.2386) (width 0.1524) (layer "F.Cu") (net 17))
 (segment (start 158.7861 125.1586) (end 158.7861 130.2386) (width 0.1524) (layer "F.Cu") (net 16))
 (segment (start 140.7761 130.2386) (end 142.2761 131.7386) (width 0.1524) (layer "F.Cu") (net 1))
 (segment (start 142.2761 131.7386) (end 142.2761 135.3186) (width 0.1524) (layer "F.Cu") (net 1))
 (segment (start 149.6661 130.2386) (end 149.6661 135.3186) (width 0.1524) (layer "F.Cu") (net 21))
 (segment (start 157.2861 135.0886) (end 157.5161 135.3186) (width 0.1524) (layer "F.Cu") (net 20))
 (segment (start 157.2861 130.2386) (end 157.2861 135.0886) (width 0.1524) (layer "F.Cu") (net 20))
 (segment (start 137.7561 95.9086) (end 140.2561 95.9086) (width 0.1524) (layer "F.Cu") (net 2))
 (segment (start 136.4461 97.2186) (end 136.4461 109.9585) (width 0.1524) (layer "F.Cu") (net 2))
 (segment (start 149.1461 137.8586) (end 143.3161 137.8586) (width 0.1524) (layer "F.Cu") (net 2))
 (segment (start 151.1661 135.8386) (end 149.1461 137.8586) (width 0.1524) (layer "F.Cu") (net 2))
 (segment (start 140.7761 135.3186) (end 137.6762 132.2187) (width 0.1524) (layer "F.Cu") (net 2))
 (segment (start 137.6762 132.2187) (end 137.6762 111.1886) (width 0.1524) (layer "F.Cu") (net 2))
 (segment (start 140.7761 135.3186) (end 143.3161 137.8586) (width 0.1524) (layer "F.Cu") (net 2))
 (segment (start 151.1661 135.3186) (end 156.0161 135.3186) (width 0.1524) (layer "F.Cu") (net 2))
 (segment (start 136.4461 109.9585) (end 137.6762 111.1886) (width 0.1524) (layer "F.Cu") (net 2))
 (segment (start 151.1661 135.3186) (end 151.1661 135.8386) (width 0.1524) (layer "F.Cu") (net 2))
 (segment (start 137.7561 95.9086) (end 136.4461 97.2186) (width 0.1524) (layer "F.Cu") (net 2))
 (segment (start 152.7021 104.8386) (end 152.9561 104.8386) (width 0.1524) (layer "F.Cu") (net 4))
 (segment (start 159.8649 102.2986) (end 161.3946 102.2986) (width 0.1524) (layer "F.Cu") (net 4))
 (segment (start 161.4905 103.9242) (end 157.602862 107.811838) (width 0.1524) (layer "F.Cu") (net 4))
 (segment (start 149.6033 104.8386) (end 149.5976 104.8386) (width 0.1524) (layer "F.Cu") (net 4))
 (segment (start 149.6033 104.8386) (end 152.7021 104.8386) (width 0.1524) (layer "F.Cu") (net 4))
 (segment (start 156.7661 107.811838) (end 156.7661 107.8632) (width 0.1524) (layer "F.Cu") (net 4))
 (segment (start 162.5573 103.6194) (end 162.2525 103.9242) (width 0.1524) (layer "F.Cu") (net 4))
 (segment (start 162.2525 103.9242) (end 161.4905 103.9242) (width 0.1524) (layer "F.Cu") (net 4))
 (segment (start 155.4961 102.2986) (end 159.8649 102.2986) (width 0.1524) (layer "F.Cu") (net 4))
 (segment (start 157.602862 107.811838) (end 156.7661 107.811838) (width 0.1524) (layer "F.Cu") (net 4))
 (segment (start 162.6646 103.5686) (end 162.5573 103.6194) (width 0.1524) (layer "F.Cu") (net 4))
 (segment (start 152.9561 104.8386) (end 155.4961 102.2986) (width 0.1524) (layer "F.Cu") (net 4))
 (segment (start 161.3946 102.2986) (end 162.6646 103.5686) (width 0.1524) (layer "F.Cu") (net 4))
 (segment (start 145.3361 104.0201) (end 146.1546 104.8386) (width 0.1524) (layer "F.Cu") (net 3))
 (segment (start 141.5261 94.6786) (end 145.3361 98.4886) (width 0.1524) (layer "F.Cu") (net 3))
 (segment (start 141.5061 94.6586) (end 141.5261 94.6786) (width 0.1524) (layer "F.Cu") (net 3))
 (segment (start 145.3361 98.4886) (end 145.3361 104.0201) (width 0.1524) (layer "F.Cu") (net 3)))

